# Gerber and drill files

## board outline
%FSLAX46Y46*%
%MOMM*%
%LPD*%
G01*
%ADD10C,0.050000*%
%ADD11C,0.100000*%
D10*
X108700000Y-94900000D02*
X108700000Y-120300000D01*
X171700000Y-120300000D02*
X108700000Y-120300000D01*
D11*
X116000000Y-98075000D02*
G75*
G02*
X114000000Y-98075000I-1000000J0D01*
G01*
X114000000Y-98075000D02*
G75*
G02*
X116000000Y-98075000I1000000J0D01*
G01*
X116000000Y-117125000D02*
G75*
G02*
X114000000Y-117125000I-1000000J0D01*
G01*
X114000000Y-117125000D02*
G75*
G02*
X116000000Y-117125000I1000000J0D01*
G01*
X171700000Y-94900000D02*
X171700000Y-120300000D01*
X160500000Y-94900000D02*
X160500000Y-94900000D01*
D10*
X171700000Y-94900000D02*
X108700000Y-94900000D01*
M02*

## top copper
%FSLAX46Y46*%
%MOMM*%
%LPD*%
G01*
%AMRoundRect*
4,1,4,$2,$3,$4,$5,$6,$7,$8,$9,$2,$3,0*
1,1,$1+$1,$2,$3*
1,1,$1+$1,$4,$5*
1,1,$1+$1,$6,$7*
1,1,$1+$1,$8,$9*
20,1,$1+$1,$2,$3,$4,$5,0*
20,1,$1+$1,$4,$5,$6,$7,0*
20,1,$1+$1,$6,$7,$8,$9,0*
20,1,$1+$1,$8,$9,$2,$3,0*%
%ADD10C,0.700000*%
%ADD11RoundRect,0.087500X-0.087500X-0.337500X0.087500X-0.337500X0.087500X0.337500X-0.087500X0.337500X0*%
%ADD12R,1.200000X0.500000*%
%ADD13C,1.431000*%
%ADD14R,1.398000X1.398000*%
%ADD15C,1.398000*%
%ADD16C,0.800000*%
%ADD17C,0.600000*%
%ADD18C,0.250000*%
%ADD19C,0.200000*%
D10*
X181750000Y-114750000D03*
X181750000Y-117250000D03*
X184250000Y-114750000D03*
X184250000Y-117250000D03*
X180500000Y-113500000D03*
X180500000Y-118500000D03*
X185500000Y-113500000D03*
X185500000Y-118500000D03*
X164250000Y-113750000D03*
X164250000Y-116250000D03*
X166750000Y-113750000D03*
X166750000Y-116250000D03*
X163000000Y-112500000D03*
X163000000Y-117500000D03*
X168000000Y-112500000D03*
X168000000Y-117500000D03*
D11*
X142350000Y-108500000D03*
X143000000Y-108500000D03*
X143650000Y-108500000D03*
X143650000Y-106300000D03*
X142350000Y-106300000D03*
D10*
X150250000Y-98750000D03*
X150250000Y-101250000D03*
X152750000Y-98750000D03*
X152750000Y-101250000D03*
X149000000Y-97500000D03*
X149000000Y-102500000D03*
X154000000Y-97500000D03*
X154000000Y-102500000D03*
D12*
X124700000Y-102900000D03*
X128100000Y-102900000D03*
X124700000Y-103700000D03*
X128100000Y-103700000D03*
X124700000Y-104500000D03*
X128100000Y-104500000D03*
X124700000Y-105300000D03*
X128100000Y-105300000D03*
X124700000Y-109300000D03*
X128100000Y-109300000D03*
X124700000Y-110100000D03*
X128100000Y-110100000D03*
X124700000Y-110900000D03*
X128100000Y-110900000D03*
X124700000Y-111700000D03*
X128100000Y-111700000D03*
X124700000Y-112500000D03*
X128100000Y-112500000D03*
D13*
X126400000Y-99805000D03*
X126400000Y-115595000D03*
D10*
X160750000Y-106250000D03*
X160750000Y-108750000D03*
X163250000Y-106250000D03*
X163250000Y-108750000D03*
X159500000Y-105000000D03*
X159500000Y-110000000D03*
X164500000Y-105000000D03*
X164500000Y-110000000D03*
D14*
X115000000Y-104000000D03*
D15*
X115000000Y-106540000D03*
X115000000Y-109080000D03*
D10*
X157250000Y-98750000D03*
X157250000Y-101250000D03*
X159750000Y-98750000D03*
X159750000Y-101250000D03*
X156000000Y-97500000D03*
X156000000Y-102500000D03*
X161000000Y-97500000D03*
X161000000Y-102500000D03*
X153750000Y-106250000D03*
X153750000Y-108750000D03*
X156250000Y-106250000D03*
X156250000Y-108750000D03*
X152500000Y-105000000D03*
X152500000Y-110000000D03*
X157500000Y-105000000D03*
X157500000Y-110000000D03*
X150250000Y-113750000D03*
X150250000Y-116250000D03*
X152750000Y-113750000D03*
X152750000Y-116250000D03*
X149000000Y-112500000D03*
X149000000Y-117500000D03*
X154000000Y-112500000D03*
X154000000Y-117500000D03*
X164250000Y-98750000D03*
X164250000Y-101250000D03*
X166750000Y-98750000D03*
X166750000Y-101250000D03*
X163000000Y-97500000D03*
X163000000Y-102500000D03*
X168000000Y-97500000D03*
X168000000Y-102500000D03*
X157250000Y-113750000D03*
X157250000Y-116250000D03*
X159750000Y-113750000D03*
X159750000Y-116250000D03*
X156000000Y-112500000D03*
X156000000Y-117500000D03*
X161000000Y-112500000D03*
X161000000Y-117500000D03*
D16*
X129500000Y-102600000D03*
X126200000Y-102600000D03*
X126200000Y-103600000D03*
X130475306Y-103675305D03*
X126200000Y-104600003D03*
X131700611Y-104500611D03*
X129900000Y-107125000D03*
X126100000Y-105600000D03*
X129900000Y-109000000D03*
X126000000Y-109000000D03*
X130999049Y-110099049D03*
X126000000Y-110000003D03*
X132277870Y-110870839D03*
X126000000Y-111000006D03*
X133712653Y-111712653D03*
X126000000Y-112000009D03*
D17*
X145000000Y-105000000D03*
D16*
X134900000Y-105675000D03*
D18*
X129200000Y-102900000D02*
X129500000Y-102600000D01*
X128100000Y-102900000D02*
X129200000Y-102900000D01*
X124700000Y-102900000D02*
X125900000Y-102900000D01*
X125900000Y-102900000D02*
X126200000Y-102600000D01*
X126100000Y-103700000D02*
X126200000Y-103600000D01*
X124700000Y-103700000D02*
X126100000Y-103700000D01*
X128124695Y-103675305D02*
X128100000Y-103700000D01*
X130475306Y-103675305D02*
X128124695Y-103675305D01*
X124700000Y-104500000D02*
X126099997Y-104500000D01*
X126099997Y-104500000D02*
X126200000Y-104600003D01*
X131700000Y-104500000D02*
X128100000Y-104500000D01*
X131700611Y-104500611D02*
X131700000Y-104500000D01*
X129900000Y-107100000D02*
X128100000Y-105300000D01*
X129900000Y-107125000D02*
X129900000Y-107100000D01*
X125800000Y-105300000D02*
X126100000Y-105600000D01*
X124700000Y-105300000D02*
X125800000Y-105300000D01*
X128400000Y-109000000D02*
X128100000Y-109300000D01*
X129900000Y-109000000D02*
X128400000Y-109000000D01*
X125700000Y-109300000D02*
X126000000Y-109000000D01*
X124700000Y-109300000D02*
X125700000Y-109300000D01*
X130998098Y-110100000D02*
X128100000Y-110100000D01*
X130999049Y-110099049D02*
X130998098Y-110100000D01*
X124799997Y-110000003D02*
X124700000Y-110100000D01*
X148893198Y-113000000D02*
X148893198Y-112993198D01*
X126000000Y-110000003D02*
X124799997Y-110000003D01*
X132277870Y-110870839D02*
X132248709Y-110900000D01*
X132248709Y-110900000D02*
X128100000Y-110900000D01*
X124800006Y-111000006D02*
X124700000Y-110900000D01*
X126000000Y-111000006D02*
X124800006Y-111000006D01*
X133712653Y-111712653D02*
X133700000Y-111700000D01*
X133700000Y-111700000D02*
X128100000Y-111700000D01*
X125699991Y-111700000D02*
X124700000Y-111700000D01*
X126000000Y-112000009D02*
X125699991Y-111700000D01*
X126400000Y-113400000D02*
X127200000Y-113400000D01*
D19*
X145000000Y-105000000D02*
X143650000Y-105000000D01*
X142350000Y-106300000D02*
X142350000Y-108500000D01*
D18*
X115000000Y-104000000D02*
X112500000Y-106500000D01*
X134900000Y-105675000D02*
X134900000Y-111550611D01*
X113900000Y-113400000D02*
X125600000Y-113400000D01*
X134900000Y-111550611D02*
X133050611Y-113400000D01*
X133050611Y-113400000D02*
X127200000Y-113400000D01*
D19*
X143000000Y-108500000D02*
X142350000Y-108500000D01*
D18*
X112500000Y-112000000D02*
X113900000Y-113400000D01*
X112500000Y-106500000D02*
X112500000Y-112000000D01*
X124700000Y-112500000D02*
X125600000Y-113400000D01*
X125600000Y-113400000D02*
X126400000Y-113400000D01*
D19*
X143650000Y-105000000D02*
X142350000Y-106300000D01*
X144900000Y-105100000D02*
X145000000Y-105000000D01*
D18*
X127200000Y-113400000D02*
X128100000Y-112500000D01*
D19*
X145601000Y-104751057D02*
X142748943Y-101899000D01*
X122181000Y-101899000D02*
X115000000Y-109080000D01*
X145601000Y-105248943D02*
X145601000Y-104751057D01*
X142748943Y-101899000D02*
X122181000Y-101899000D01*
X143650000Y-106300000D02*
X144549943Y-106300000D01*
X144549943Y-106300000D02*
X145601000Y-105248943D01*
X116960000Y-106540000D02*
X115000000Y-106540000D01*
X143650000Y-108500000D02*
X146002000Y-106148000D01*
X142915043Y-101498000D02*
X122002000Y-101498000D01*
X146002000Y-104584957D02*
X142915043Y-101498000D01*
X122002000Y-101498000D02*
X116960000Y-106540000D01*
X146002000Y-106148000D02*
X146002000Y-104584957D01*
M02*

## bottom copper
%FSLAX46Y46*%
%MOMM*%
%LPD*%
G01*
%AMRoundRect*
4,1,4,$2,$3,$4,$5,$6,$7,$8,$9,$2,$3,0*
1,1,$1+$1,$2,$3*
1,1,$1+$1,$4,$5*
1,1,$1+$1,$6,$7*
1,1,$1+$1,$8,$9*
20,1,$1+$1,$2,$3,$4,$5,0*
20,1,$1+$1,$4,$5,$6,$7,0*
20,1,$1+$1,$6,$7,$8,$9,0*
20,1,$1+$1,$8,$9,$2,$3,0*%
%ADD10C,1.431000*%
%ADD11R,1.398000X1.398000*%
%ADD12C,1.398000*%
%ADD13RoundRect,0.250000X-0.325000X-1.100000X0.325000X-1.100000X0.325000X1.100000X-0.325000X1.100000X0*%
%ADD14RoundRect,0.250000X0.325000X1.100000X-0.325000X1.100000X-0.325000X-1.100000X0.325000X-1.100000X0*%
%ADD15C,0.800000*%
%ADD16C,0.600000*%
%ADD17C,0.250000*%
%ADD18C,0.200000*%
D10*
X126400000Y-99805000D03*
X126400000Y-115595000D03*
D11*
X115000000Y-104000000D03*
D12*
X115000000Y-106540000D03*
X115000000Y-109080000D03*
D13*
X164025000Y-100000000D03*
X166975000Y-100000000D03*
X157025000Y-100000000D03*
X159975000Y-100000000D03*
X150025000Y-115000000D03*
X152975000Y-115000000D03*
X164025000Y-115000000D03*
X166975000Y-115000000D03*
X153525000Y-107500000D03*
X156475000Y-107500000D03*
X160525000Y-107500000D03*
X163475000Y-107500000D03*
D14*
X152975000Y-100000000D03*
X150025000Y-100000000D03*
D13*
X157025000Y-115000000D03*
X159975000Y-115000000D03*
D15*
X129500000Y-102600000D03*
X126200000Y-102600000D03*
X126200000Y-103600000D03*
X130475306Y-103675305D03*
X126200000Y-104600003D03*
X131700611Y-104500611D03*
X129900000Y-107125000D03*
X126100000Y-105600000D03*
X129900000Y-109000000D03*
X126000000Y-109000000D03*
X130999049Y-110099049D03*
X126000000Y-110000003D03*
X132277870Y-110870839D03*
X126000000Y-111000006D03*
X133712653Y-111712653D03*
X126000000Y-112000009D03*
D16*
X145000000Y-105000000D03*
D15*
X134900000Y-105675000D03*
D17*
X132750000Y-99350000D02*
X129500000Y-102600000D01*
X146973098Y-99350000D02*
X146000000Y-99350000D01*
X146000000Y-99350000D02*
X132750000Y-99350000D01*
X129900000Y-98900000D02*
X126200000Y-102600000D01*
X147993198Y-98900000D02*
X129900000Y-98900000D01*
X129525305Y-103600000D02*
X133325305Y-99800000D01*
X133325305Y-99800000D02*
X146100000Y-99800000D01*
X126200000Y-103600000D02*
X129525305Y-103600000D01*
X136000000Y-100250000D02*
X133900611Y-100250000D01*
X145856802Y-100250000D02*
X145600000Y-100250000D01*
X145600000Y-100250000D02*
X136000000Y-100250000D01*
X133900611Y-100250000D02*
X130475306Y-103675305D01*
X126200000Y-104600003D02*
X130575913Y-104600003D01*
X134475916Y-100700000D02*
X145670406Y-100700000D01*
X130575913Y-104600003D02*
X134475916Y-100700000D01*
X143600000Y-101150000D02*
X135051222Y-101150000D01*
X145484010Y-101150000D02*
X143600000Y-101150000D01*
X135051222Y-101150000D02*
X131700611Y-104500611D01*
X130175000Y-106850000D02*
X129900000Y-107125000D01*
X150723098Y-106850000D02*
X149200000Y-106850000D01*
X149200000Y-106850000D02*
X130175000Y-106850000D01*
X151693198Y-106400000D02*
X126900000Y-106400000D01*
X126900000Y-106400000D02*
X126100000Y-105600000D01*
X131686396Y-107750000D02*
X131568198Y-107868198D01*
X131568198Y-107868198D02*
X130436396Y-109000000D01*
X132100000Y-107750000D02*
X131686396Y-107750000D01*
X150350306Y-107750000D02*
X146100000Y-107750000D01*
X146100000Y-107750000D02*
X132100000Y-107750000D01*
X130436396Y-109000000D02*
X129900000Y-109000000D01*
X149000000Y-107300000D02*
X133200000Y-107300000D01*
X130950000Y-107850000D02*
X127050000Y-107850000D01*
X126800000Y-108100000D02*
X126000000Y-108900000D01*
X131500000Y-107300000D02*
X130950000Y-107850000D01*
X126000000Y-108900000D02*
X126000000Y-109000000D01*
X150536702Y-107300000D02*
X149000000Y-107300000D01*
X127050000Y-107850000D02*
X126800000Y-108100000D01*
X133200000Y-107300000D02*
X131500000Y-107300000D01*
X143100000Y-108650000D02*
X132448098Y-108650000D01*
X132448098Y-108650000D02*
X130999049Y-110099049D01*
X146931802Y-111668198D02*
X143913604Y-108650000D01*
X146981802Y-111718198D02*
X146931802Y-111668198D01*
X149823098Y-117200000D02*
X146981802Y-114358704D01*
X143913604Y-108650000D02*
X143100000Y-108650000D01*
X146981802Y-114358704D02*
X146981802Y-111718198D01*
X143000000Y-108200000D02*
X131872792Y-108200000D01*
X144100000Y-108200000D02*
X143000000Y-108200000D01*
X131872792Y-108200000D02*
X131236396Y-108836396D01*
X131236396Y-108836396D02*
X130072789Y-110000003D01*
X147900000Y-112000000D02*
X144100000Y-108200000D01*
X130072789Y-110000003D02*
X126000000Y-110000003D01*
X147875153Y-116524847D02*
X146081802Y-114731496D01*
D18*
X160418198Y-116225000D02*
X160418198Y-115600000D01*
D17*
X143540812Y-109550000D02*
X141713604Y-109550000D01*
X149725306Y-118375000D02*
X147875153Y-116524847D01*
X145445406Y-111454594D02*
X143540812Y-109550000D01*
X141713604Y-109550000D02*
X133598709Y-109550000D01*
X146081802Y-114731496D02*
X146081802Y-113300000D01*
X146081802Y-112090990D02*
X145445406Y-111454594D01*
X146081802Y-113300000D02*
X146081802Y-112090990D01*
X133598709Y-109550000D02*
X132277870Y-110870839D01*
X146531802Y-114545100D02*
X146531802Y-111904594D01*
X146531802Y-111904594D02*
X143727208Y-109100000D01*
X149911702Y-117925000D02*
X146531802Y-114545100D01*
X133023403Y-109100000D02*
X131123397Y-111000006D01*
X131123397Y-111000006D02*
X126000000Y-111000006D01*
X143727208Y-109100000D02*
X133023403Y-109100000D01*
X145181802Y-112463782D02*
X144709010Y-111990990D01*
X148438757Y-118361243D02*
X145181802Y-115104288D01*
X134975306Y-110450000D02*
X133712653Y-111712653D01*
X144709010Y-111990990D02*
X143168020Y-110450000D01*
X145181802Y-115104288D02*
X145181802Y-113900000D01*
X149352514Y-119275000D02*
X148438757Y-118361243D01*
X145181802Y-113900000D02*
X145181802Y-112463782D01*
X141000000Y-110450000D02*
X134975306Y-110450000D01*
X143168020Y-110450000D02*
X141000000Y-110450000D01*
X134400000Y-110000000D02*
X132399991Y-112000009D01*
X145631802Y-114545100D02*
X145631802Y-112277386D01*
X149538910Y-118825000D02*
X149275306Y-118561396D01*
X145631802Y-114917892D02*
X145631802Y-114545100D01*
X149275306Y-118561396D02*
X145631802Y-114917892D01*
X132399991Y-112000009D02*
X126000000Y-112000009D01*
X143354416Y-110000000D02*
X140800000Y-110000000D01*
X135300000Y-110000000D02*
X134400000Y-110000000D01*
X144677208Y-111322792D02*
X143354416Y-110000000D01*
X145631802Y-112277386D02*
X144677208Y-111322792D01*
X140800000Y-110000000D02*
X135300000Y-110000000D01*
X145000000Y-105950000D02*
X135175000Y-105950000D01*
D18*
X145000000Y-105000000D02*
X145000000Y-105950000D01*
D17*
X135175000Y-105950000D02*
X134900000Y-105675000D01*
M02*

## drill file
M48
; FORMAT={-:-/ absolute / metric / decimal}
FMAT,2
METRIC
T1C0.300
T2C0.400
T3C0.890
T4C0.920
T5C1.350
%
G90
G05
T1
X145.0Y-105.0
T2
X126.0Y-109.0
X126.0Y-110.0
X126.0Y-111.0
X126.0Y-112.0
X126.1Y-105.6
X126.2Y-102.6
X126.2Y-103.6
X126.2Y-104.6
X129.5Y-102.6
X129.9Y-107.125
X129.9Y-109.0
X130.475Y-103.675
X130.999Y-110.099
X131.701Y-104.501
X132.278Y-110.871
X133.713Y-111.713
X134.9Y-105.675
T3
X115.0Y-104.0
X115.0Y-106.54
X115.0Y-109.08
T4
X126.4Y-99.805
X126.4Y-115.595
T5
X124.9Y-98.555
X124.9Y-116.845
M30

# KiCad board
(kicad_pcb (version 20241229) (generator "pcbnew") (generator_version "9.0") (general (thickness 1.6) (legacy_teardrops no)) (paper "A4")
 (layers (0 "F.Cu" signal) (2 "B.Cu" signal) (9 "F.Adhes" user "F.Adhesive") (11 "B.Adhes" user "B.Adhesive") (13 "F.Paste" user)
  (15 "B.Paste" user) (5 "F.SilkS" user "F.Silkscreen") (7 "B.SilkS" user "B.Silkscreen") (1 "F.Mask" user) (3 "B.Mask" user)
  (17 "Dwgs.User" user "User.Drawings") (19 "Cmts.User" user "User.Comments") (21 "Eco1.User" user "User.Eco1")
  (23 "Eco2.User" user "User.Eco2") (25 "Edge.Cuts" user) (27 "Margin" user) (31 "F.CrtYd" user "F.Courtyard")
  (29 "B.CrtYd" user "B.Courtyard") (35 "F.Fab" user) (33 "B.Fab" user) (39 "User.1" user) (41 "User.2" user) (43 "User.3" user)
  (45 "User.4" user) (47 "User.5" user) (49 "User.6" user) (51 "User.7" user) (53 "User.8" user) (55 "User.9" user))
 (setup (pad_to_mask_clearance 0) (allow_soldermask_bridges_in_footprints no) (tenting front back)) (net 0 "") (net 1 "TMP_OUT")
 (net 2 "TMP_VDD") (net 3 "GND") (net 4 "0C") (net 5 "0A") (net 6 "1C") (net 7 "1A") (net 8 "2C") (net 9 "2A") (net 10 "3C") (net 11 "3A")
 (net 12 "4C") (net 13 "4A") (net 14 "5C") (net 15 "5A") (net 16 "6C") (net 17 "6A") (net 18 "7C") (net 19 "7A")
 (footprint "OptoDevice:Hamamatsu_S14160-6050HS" (layer "F.Cu") (at 183 116)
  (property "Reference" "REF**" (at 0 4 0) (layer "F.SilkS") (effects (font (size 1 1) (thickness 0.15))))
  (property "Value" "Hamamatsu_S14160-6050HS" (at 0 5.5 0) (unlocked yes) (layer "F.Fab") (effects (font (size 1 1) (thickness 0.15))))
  (pad "A" smd circle (at -1.25 -1.25) (size 0.7 0.7) (layers "F.Cu" "F.Mask" "F.Paste"))
  (pad "A" smd circle (at -1.25 1.25) (size 0.7 0.7) (layers "F.Cu" "F.Mask" "F.Paste"))
  (pad "A" smd circle (at 1.25 -1.25) (size 0.7 0.7) (layers "F.Cu" "F.Mask" "F.Paste"))
  (pad "A" smd circle (at 1.25 1.25) (size 0.7 0.7) (layers "F.Cu" "F.Mask" "F.Paste"))
  (pad "K" smd circle (at -2.5 -2.5) (size 0.7 0.7) (layers "F.Cu" "F.Mask" "F.Paste"))
  (pad "K" smd circle (at -2.5 2.5) (size 0.7 0.7) (layers "F.Cu" "F.Mask" "F.Paste"))
  (pad "K" smd circle (at 2.5 -2.5) (size 0.7 0.7) (layers "F.Cu" "F.Mask" "F.Paste"))
  (pad "K" smd circle (at 2.5 2.5) (size 0.7 0.7) (layers "F.Cu" "F.Mask" "F.Paste")))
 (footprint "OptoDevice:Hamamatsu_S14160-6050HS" (layer "F.Cu") (at 165.5 115)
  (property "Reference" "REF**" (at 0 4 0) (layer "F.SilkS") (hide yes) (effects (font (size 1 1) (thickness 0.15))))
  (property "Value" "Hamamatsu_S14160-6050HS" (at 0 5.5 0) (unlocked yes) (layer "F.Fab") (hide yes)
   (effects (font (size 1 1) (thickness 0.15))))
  (pad "A" smd circle (at -1.25 -1.25) (size 0.7 0.7) (layers "F.Cu" "F.Mask" "F.Paste"))
  (pad "A" smd circle (at -1.25 1.25) (size 0.7 0.7) (layers "F.Cu" "F.Mask" "F.Paste"))
  (pad "A" smd circle (at 1.25 -1.25) (size 0.7 0.7) (layers "F.Cu" "F.Mask" "F.Paste"))
  (pad "A" smd circle (at 1.25 1.25) (size 0.7 0.7) (layers "F.Cu" "F.Mask" "F.Paste"))
  (pad "K" smd circle (at -2.5 -2.5) (size 0.7 0.7) (layers "F.Cu" "F.Mask" "F.Paste"))
  (pad "K" smd circle (at -2.5 2.5) (size 0.7 0.7) (layers "F.Cu" "F.Mask" "F.Paste"))
  (pad "K" smd circle (at 2.5 -2.5) (size 0.7 0.7) (layers "F.Cu" "F.Mask" "F.Paste"))
  (pad "K" smd circle (at 2.5 2.5) (size 0.7 0.7) (layers "F.Cu" "F.Mask" "F.Paste")))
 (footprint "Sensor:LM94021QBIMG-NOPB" (layer "F.Cu") (at 143 107.4)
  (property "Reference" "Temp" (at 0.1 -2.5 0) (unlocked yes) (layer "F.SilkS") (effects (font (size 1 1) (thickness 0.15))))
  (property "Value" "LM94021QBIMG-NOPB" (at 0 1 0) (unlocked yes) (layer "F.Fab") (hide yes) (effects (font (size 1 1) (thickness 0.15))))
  (pad "1" smd roundrect (at -0.65 1.1) (size 0.35 0.85) (layers "F.Cu" "F.Mask" "F.Paste") (roundrect_rratio 0.25))
  (pad "2" smd roundrect (at 0 1.1) (size 0.35 0.85) (layers "F.Cu" "F.Mask" "F.Paste") (roundrect_rratio 0.25))
  (pad "3" smd roundrect (at 0.65 1.1) (size 0.35 0.85) (layers "F.Cu" "F.Mask" "F.Paste") (roundrect_rratio 0.25) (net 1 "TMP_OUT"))
  (pad "4" smd roundrect (at 0.65 -1.1) (size 0.35 0.85) (layers "F.Cu" "F.Mask" "F.Paste") (roundrect_rratio 0.25) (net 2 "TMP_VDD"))
  (pad "5" smd roundrect (at -0.65 -1.1) (size 0.35 0.85) (layers "F.Cu" "F.Mask" "F.Paste") (roundrect_rratio 0.25) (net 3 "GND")))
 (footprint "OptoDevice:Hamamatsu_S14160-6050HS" (layer "F.Cu") (at 151.5 100)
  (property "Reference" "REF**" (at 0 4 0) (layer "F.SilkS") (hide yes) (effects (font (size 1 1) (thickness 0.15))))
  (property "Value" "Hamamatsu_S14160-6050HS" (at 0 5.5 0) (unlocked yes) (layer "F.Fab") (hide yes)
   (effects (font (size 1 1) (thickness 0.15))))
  (pad "A" smd circle (at -1.25 -1.25) (size 0.7 0.7) (layers "F.Cu" "F.Mask" "F.Paste") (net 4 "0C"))
  (pad "A" smd circle (at -1.25 1.25) (size 0.7 0.7) (layers "F.Cu" "F.Mask" "F.Paste") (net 4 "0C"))
  (pad "A" smd circle (at 1.25 -1.25) (size 0.7 0.7) (layers "F.Cu" "F.Mask" "F.Paste") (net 4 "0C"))
  (pad "A" smd circle (at 1.25 1.25) (size 0.7 0.7) (layers "F.Cu" "F.Mask" "F.Paste") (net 4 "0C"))
  (pad "K" smd circle (at -2.5 -2.5) (size 0.7 0.7) (layers "F.Cu" "F.Mask" "F.Paste") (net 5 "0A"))
  (pad "K" smd circle (at -2.5 2.5) (size 0.7 0.7) (layers "F.Cu" "F.Mask" "F.Paste") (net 5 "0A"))
  (pad "K" smd circle (at 2.5 -2.5) (size 0.7 0.7) (layers "F.Cu" "F.Mask" "F.Paste") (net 5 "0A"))
  (pad "K" smd circle (at 2.5 2.5) (size 0.7 0.7) (layers "F.Cu" "F.Mask" "F.Paste") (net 5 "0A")))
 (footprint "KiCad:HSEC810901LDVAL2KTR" (layer "F.Cu") (at 126.4 107.7 -90)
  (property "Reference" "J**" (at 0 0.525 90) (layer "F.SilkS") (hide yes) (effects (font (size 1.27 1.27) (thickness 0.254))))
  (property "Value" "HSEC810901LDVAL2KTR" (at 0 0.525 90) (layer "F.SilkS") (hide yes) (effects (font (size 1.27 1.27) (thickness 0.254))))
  (pad "" np_thru_hole circle (at -9.145 1.5 270) (size 1.35 1.35) (drill 1.35) (layers "*.Cu" "*.Mask"))
  (pad "" np_thru_hole circle (at 9.145 1.5 270) (size 1.35 1.35) (drill 1.35) (layers "*.Cu" "*.Mask"))
  (pad "1" smd rect (at -4.8 1.7 270) (size 0.5 1.2) (layers "F.Cu" "F.Mask" "F.Paste") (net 4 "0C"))
  (pad "2" smd rect (at -4.8 -1.7 270) (size 0.5 1.2) (layers "F.Cu" "F.Mask" "F.Paste") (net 5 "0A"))
  (pad "3" smd rect (at -4 1.7 270) (size 0.5 1.2) (layers "F.Cu" "F.Mask" "F.Paste") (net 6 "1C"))
  (pad "4" smd rect (at -4 -1.7 270) (size 0.5 1.2) (layers "F.Cu" "F.Mask" "F.Paste") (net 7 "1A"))
  (pad "5" smd rect (at -3.2 1.7 270) (size 0.5 1.2) (layers "F.Cu" "F.Mask" "F.Paste") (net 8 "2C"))
  (pad "6" smd rect (at -3.2 -1.7 270) (size 0.5 1.2) (layers "F.Cu" "F.Mask" "F.Paste") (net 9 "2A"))
  (pad "7" smd rect (at -2.4 1.7 270) (size 0.5 1.2) (layers "F.Cu" "F.Mask" "F.Paste") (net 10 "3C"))
  (pad "8" smd rect (at -2.4 -1.7 270) (size 0.5 1.2) (layers "F.Cu" "F.Mask" "F.Paste") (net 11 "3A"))
  (pad "9" smd rect (at 1.6 1.7 270) (size 0.5 1.2) (layers "F.Cu" "F.Mask" "F.Paste") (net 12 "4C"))
  (pad "10" smd rect (at 1.6 -1.7 270) (size 0.5 1.2) (layers "F.Cu" "F.Mask" "F.Paste") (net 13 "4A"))
  (pad "11" smd rect (at 2.4 1.7 270) (size 0.5 1.2) (layers "F.Cu" "F.Mask" "F.Paste") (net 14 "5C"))
  (pad "12" smd rect (at 2.4 -1.7 270) (size 0.5 1.2) (layers "F.Cu" "F.Mask" "F.Paste") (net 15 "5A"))
  (pad "13" smd rect (at 3.2 1.7 270) (size 0.5 1.2) (layers "F.Cu" "F.Mask" "F.Paste") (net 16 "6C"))
  (pad "14" smd rect (at 3.2 -1.7 270) (size 0.5 1.2) (layers "F.Cu" "F.Mask" "F.Paste") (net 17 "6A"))
  (pad "15" smd rect (at 4 1.7 270) (size 0.5 1.2) (layers "F.Cu" "F.Mask" "F.Paste") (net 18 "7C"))
  (pad "16" smd rect (at 4 -1.7 270) (size 0.5 1.2) (layers "F.Cu" "F.Mask" "F.Paste") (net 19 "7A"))
  (pad "17" smd rect (at 4.8 1.7 270) (size 0.5 1.2) (layers "F.Cu" "F.Mask" "F.Paste") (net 3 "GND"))
  (pad "18" smd rect (at 4.8 -1.7 270) (size 0.5 1.2) (layers "F.Cu" "F.Mask" "F.Paste") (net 3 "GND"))
  (pad "MH1" thru_hole circle (at -7.895 0 270) (size 1.431 1.431) (drill 0.92) (layers "*.Cu" "*.Mask") (remove_unused_layers no))
  (pad "MH2" thru_hole circle (at 7.895 0 270) (size 1.431 1.431) (drill 0.92) (layers "*.Cu" "*.Mask") (remove_unused_layers no)))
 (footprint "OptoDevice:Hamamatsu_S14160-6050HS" (layer "F.Cu") (at 162 107.5)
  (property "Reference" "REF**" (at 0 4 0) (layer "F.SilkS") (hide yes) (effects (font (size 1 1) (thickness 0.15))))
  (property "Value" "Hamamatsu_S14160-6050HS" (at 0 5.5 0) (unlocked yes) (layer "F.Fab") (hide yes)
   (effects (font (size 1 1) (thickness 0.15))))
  (pad "A" smd circle (at -1.25 -1.25) (size 0.7 0.7) (layers "F.Cu" "F.Mask" "F.Paste"))
  (pad "A" smd circle (at -1.25 1.25) (size 0.7 0.7) (layers "F.Cu" "F.Mask" "F.Paste"))
  (pad "A" smd circle (at 1.25 -1.25) (size 0.7 0.7) (layers "F.Cu" "F.Mask" "F.Paste"))
  (pad "A" smd circle (at 1.25 1.25) (size 0.7 0.7) (layers "F.Cu" "F.Mask" "F.Paste"))
  (pad "K" smd circle (at -2.5 -2.5) (size 0.7 0.7) (layers "F.Cu" "F.Mask" "F.Paste"))
  (pad "K" smd circle (at -2.5 2.5) (size 0.7 0.7) (layers "F.Cu" "F.Mask" "F.Paste"))
  (pad "K" smd circle (at 2.5 -2.5) (size 0.7 0.7) (layers "F.Cu" "F.Mask" "F.Paste"))
  (pad "K" smd circle (at 2.5 2.5) (size 0.7 0.7) (layers "F.Cu" "F.Mask" "F.Paste")))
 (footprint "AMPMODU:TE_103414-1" (layer "F.Cu") (at 115 106.54 -90)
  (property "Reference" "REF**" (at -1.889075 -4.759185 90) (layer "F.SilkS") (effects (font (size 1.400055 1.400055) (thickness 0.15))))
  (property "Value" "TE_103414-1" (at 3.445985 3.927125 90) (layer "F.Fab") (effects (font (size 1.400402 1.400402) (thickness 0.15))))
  (pad "1" thru_hole rect (at -2.54 0 270) (size 1.398 1.398) (drill 0.89) (layers "*.Cu" "*.Mask") (remove_unused_layers no) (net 3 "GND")
   (solder_mask_margin 0.102))
  (pad "2" thru_hole circle (at 0 0 270) (size 1.398 1.398) (drill 0.89) (layers "*.Cu" "*.Mask") (remove_unused_layers no)
   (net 1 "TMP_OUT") (solder_mask_margin 0.102))
  (pad "3" thru_hole circle (at 2.54 0 270) (size 1.398 1.398) (drill 0.89) (layers "*.Cu" "*.Mask") (remove_unused_layers no)
   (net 2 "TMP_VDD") (solder_mask_margin 0.102)))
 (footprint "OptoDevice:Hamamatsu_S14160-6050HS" (layer "F.Cu") (at 158.5 100)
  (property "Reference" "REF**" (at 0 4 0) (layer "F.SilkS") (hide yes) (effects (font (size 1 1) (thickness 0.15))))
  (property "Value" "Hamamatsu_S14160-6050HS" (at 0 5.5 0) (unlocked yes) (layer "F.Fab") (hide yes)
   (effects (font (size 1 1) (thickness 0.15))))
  (pad "A" smd circle (at -1.25 -1.25) (size 0.7 0.7) (layers "F.Cu" "F.Mask" "F.Paste") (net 6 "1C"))
  (pad "A" smd circle (at -1.25 1.25) (size 0.7 0.7) (layers "F.Cu" "F.Mask" "F.Paste") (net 6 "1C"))
  (pad "A" smd circle (at 1.25 -1.25) (size 0.7 0.7) (layers "F.Cu" "F.Mask" "F.Paste") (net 6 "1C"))
  (pad "A" smd circle (at 1.25 1.25) (size 0.7 0.7) (layers "F.Cu" "F.Mask" "F.Paste") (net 6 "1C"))
  (pad "K" smd circle (at -2.5 -2.5) (size 0.7 0.7) (layers "F.Cu" "F.Mask" "F.Paste") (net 7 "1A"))
  (pad "K" smd circle (at -2.5 2.5) (size 0.7 0.7) (layers "F.Cu" "F.Mask" "F.Paste") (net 7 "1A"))
  (pad "K" smd circle (at 2.5 -2.5) (size 0.7 0.7) (layers "F.Cu" "F.Mask" "F.Paste") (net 7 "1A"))
  (pad "K" smd circle (at 2.5 2.5) (size 0.7 0.7) (layers "F.Cu" "F.Mask" "F.Paste") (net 7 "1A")))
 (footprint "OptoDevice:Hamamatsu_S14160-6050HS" (layer "F.Cu") (at 155 107.5)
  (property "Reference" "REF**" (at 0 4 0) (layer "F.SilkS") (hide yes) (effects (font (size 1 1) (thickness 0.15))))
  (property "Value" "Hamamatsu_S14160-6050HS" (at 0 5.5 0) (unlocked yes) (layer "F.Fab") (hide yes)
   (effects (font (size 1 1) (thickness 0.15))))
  (pad "A" smd circle (at -1.25 -1.25) (size 0.7 0.7) (layers "F.Cu" "F.Mask" "F.Paste") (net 10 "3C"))
  (pad "A" smd circle (at -1.25 1.25) (size 0.7 0.7) (layers "F.Cu" "F.Mask" "F.Paste") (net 10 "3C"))
  (pad "A" smd circle (at 1.25 -1.25) (size 0.7 0.7) (layers "F.Cu" "F.Mask" "F.Paste") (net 10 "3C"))
  (pad "A" smd circle (at 1.25 1.25) (size 0.7 0.7) (layers "F.Cu" "F.Mask" "F.Paste") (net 10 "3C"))
  (pad "K" smd circle (at -2.5 -2.5) (size 0.7 0.7) (layers "F.Cu" "F.Mask" "F.Paste") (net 11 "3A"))
  (pad "K" smd circle (at -2.5 2.5) (size 0.7 0.7) (layers "F.Cu" "F.Mask" "F.Paste") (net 11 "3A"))
  (pad "K" smd circle (at 2.5 -2.5) (size 0.7 0.7) (layers "F.Cu" "F.Mask" "F.Paste") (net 11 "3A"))
  (pad "K" smd circle (at 2.5 2.5) (size 0.7 0.7) (layers "F.Cu" "F.Mask" "F.Paste") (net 11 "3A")))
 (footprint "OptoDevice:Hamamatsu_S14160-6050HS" (layer "F.Cu") (at 151.5 115)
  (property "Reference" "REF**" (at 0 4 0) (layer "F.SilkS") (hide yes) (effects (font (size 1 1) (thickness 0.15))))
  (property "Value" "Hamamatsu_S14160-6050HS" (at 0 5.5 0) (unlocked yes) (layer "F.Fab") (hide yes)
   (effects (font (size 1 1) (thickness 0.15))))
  (pad "A" smd circle (at -1.25 -1.25) (size 0.7 0.7) (layers "F.Cu" "F.Mask" "F.Paste"))
  (pad "A" smd circle (at -1.25 1.25) (size 0.7 0.7) (layers "F.Cu" "F.Mask" "F.Paste"))
  (pad "A" smd circle (at 1.25 -1.25) (size 0.7 0.7) (layers "F.Cu" "F.Mask" "F.Paste"))
  (pad "A" smd circle (at 1.25 1.25) (size 0.7 0.7) (layers "F.Cu" "F.Mask" "F.Paste"))
  (pad "K" smd circle (at -2.5 -2.5) (size 0.7 0.7) (layers "F.Cu" "F.Mask" "F.Paste"))
  (pad "K" smd circle (at -2.5 2.5) (size 0.7 0.7) (layers "F.Cu" "F.Mask" "F.Paste"))
  (pad "K" smd circle (at 2.5 -2.5) (size 0.7 0.7) (layers "F.Cu" "F.Mask" "F.Paste"))
  (pad "K" smd circle (at 2.5 2.5) (size 0.7 0.7) (layers "F.Cu" "F.Mask" "F.Paste")))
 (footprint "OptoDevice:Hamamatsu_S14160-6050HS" (layer "F.Cu") (at 165.5 100)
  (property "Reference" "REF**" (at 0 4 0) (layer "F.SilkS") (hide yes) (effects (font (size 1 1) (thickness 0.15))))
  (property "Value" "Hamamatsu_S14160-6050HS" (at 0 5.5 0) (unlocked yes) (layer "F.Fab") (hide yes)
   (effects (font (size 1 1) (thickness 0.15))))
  (pad "A" smd circle (at -1.25 -1.25) (size 0.7 0.7) (layers "F.Cu" "F.Mask" "F.Paste") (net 8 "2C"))
  (pad "A" smd circle (at -1.25 1.25) (size 0.7 0.7) (layers "F.Cu" "F.Mask" "F.Paste") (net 8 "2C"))
  (pad "A" smd circle (at 1.25 -1.25) (size 0.7 0.7) (layers "F.Cu" "F.Mask" "F.Paste") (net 8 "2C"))
  (pad "A" smd circle (at 1.25 1.25) (size 0.7 0.7) (layers "F.Cu" "F.Mask" "F.Paste") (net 8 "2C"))
  (pad "K" smd circle (at -2.5 -2.5) (size 0.7 0.7) (layers "F.Cu" "F.Mask" "F.Paste") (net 9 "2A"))
  (pad "K" smd circle (at -2.5 2.5) (size 0.7 0.7) (layers "F.Cu" "F.Mask" "F.Paste") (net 9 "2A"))
  (pad "K" smd circle (at 2.5 -2.5) (size 0.7 0.7) (layers "F.Cu" "F.Mask" "F.Paste") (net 9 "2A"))
  (pad "K" smd circle (at 2.5 2.5) (size 0.7 0.7) (layers "F.Cu" "F.Mask" "F.Paste") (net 9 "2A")))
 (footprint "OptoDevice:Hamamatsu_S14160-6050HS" (layer "F.Cu") (at 158.5 115)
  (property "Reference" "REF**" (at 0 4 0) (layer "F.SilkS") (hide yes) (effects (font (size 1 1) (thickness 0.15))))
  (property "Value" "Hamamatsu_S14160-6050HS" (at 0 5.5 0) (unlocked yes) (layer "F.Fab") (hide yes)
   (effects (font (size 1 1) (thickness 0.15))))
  (pad "A" smd circle (at -1.25 -1.25) (size 0.7 0.7) (layers "F.Cu" "F.Mask" "F.Paste"))
  (pad "A" smd circle (at -1.25 1.25) (size 0.7 0.7) (layers "F.Cu" "F.Mask" "F.Paste"))
  (pad "A" smd circle (at 1.25 -1.25) (size 0.7 0.7) (layers "F.Cu" "F.Mask" "F.Paste"))
  (pad "A" smd circle (at 1.25 1.25) (size 0.7 0.7) (layers "F.Cu" "F.Mask" "F.Paste"))
  (pad "K" smd circle (at -2.5 -2.5) (size 0.7 0.7) (layers "F.Cu" "F.Mask" "F.Paste"))
  (pad "K" smd circle (at -2.5 2.5) (size 0.7 0.7) (layers "F.Cu" "F.Mask" "F.Paste"))
  (pad "K" smd circle (at 2.5 -2.5) (size 0.7 0.7) (layers "F.Cu" "F.Mask" "F.Paste"))
  (pad "K" smd circle (at 2.5 2.5) (size 0.7 0.7) (layers "F.Cu" "F.Mask" "F.Paste")))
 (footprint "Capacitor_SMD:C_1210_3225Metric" (layer "B.Cu") (at 165.5 100)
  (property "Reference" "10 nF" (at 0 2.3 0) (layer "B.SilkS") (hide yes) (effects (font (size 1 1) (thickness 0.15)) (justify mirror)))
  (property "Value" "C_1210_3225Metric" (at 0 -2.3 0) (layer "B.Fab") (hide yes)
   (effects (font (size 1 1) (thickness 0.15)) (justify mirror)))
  (pad "1" smd roundrect (at -1.475 0) (size 1.15 2.7) (layers "B.Cu" "B.Mask" "B.Paste") (roundrect_rratio 0.2173913043) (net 3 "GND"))
  (pad "2" smd roundrect (at 1.475 0) (size 1.15 2.7) (layers "B.Cu" "B.Mask" "B.Paste") (roundrect_rratio 0.2173913043) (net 9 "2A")))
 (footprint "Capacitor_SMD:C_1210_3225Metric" (layer "B.Cu") (at 158.5 100)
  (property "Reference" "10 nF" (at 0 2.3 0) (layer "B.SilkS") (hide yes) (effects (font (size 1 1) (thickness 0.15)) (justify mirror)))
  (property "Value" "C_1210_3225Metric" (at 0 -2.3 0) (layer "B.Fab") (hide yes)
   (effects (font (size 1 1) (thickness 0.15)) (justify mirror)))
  (pad "1" smd roundrect (at -1.475 0) (size 1.15 2.7) (layers "B.Cu" "B.Mask" "B.Paste") (roundrect_rratio 0.2173913043) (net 3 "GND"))
  (pad "2" smd roundrect (at 1.475 0) (size 1.15 2.7) (layers "B.Cu" "B.Mask" "B.Paste") (roundrect_rratio 0.2173913043) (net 7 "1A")))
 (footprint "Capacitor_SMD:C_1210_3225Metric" (layer "B.Cu") (at 151.5 115)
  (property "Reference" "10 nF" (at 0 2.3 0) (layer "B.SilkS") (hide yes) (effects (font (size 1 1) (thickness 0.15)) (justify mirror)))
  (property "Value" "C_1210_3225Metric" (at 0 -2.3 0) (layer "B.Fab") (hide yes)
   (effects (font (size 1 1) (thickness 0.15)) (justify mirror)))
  (pad "1" smd roundrect (at -1.475 0) (size 1.15 2.7) (layers "B.Cu" "B.Mask" "B.Paste") (roundrect_rratio 0.2173913043) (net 3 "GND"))
  (pad "2" smd roundrect (at 1.475 0) (size 1.15 2.7) (layers "B.Cu" "B.Mask" "B.Paste") (roundrect_rratio 0.2173913043) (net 15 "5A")))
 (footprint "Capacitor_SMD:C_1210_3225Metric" (layer "B.Cu") (at 165.5 115)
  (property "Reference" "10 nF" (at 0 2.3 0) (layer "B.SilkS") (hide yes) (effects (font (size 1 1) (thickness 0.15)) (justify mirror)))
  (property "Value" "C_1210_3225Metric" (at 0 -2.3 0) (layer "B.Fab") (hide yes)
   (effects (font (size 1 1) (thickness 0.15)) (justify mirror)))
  (pad "1" smd roundrect (at -1.475 0) (size 1.15 2.7) (layers "B.Cu" "B.Mask" "B.Paste") (roundrect_rratio 0.2173913043) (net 3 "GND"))
  (pad "2" smd roundrect (at 1.475 0) (size 1.15 2.7) (layers "B.Cu" "B.Mask" "B.Paste") (roundrect_rratio 0.2173913043) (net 19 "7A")))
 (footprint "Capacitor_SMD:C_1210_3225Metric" (layer "B.Cu") (at 155 107.5)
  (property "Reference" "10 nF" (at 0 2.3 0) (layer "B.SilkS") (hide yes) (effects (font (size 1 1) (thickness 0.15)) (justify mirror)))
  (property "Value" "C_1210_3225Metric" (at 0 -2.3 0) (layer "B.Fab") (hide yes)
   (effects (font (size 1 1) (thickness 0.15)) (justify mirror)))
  (pad "1" smd roundrect (at -1.475 0) (size 1.15 2.7) (layers "B.Cu" "B.Mask" "B.Paste") (roundrect_rratio 0.2173913043) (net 3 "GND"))
  (pad "2" smd roundrect (at 1.475 0) (size 1.15 2.7) (layers "B.Cu" "B.Mask" "B.Paste") (roundrect_rratio 0.2173913043) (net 11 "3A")))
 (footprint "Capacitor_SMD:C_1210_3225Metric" (layer "B.Cu") (at 162 107.5)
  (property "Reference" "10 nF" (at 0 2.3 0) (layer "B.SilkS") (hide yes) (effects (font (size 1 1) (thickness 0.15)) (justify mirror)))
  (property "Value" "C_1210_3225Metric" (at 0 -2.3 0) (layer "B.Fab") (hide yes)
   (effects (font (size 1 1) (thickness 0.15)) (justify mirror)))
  (pad "1" smd roundrect (at -1.475 0) (size 1.15 2.7) (layers "B.Cu" "B.Mask" "B.Paste") (roundrect_rratio 0.2173913043) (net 3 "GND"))
  (pad "2" smd roundrect (at 1.475 0) (size 1.15 2.7) (layers "B.Cu" "B.Mask" "B.Paste") (roundrect_rratio 0.2173913043) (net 13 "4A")))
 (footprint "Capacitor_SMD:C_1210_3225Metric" (layer "B.Cu") (at 151.5 100 180)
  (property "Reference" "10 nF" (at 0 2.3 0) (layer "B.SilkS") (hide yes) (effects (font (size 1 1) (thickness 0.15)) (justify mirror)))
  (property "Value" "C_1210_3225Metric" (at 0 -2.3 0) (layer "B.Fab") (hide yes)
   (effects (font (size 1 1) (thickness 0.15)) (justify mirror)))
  (pad "1" smd roundrect (at -1.475 0 180) (size 1.15 2.7) (layers "B.Cu" "B.Mask" "B.Paste") (roundrect_rratio 0.2173913043) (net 5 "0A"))
  (pad "2" smd roundrect (at 1.475 0 180) (size 1.15 2.7) (layers "B.Cu" "B.Mask" "B.Paste") (roundrect_rratio 0.2173913043) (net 3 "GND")))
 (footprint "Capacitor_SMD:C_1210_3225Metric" (layer "B.Cu") (at 158.5 115)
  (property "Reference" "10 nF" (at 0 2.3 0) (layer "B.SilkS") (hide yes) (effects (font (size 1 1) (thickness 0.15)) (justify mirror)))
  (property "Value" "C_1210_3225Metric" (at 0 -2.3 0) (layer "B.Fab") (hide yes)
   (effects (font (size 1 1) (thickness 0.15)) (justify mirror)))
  (pad "1" smd roundrect (at -1.475 0) (size 1.15 2.7) (layers "B.Cu" "B.Mask" "B.Paste") (roundrect_rratio 0.2173913043) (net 3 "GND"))
  (pad "2" smd roundrect (at 1.475 0) (size 1.15 2.7) (layers "B.Cu" "B.Mask" "B.Paste") (roundrect_rratio 0.2173913043) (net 17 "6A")))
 (gr_line (start 108.7 94.9) (end 108.7 120.3) (stroke (width 0.05) (type default)) (layer "Edge.Cuts"))
 (gr_line (start 171.7 120.3) (end 108.7 120.3) (stroke (width 0.05) (type solid)) (layer "Edge.Cuts"))
 (gr_circle (center 115 98.075) (end 116 98.075) (stroke (width 0.1) (type solid)) (fill no) (layer "Edge.Cuts"))
 (gr_circle (center 115 117.125) (end 116 117.125) (stroke (width 0.1) (type solid)) (fill no) (layer "Edge.Cuts"))
 (gr_line (start 171.7 94.9) (end 171.7 120.3) (stroke (width 0.1) (type default)) (layer "Edge.Cuts"))
 (gr_line (start 160.5 94.9) (end 160.5 94.9) (stroke (width 0.1) (type default)) (layer "Edge.Cuts"))
 (gr_line (start 171.7 94.9) (end 108.7 94.9) (stroke (width 0.05) (type solid)) (layer "Edge.Cuts"))
 (segment (start 129.2 102.9) (end 129.5 102.6) (width 0.25) (layer "F.Cu") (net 5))
 (segment (start 128.1 102.9) (end 129.2 102.9) (width 0.25) (layer "F.Cu") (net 5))
 (via (at 129.5 102.6) (size 0.8) (drill 0.4) (layers "F.Cu" "B.Cu") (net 5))
 (segment (start 132.75 99.35) (end 129.5 102.6) (width 0.25) (layer "B.Cu") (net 5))
 (segment (start 146.973098 99.35) (end 146 99.35) (width 0.25) (layer "B.Cu") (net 5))
 (segment (start 146 99.35) (end 132.75 99.35) (width 0.25) (layer "B.Cu") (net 5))
 (segment (start 124.7 102.9) (end 125.9 102.9) (width 0.25) (layer "F.Cu") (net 4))
 (segment (start 125.9 102.9) (end 126.2 102.6) (width 0.25) (layer "F.Cu") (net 4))
 (via (at 126.2 102.6) (size 0.8) (drill 0.4) (layers "F.Cu" "B.Cu") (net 4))
 (segment (start 129.9 98.9) (end 126.2 102.6) (width 0.25) (layer "B.Cu") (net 4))
 (segment (start 147.993198 98.9) (end 129.9 98.9) (width 0.25) (layer "B.Cu") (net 4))
 (segment (start 126.1 103.7) (end 126.2 103.6) (width 0.25) (layer "F.Cu") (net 6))
 (segment (start 124.7 103.7) (end 126.1 103.7) (width 0.25) (layer "F.Cu") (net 6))
 (via (at 126.2 103.6) (size 0.8) (drill 0.4) (layers "F.Cu" "B.Cu") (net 6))
 (segment (start 129.525305 103.6) (end 133.325305 99.8) (width 0.25) (layer "B.Cu") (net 6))
 (segment (start 133.325305 99.8) (end 146.1 99.8) (width 0.25) (layer "B.Cu") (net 6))
 (segment (start 126.2 103.6) (end 129.525305 103.6) (width 0.25) (layer "B.Cu") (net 6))
 (segment (start 128.124695 103.675305) (end 128.1 103.7) (width 0.25) (layer "F.Cu") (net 7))
 (segment (start 130.475306 103.675305) (end 128.124695 103.675305) (width 0.25) (layer "F.Cu") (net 7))
 (via (at 130.475306 103.675305) (size 0.8) (drill 0.4) (layers "F.Cu" "B.Cu") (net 7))
 (segment (start 136 100.25) (end 133.900611 100.25) (width 0.25) (layer "B.Cu") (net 7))
 (segment (start 145.856802 100.25) (end 145.6 100.25) (width 0.25) (layer "B.Cu") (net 7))
 (segment (start 145.6 100.25) (end 136 100.25) (width 0.25) (layer "B.Cu") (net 7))
 (segment (start 133.900611 100.25) (end 130.475306 103.675305) (width 0.25) (layer "B.Cu") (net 7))
 (segment (start 124.7 104.5) (end 126.099997 104.5) (width 0.25) (layer "F.Cu") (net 8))
 (segment (start 126.099997 104.5) (end 126.2 104.600003) (width 0.25) (layer "F.Cu") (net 8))
 (via (at 126.2 104.600003) (size 0.8) (drill 0.4) (layers "F.Cu" "B.Cu") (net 8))
 (segment (start 126.2 104.600003) (end 130.575913 104.600003) (width 0.25) (layer "B.Cu") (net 8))
 (segment (start 134.475916 100.7) (end 145.670406 100.7) (width 0.25) (layer "B.Cu") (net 8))
 (segment (start 130.575913 104.600003) (end 134.475916 100.7) (width 0.25) (layer "B.Cu") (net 8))
 (segment (start 131.7 104.5) (end 128.1 104.5) (width 0.25) (layer "F.Cu") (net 9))
 (segment (start 131.700611 104.500611) (end 131.7 104.5) (width 0.25) (layer "F.Cu") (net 9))
 (via (at 131.700611 104.500611) (size 0.8) (drill 0.4) (layers "F.Cu" "B.Cu") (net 9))
 (segment (start 143.6 101.15) (end 135.051222 101.15) (width 0.25) (layer "B.Cu") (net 9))
 (segment (start 145.48401 101.15) (end 143.6 101.15) (width 0.25) (layer "B.Cu") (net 9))
 (segment (start 135.051222 101.15) (end 131.700611 104.500611) (width 0.25) (layer "B.Cu") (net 9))
 (segment (start 129.9 107.1) (end 128.1 105.3) (width 0.25) (layer "F.Cu") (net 11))
 (segment (start 129.9 107.125) (end 129.9 107.1) (width 0.25) (layer "F.Cu") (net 11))
 (via (at 129.9 107.125) (size 0.8) (drill 0.4) (layers "F.Cu" "B.Cu") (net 11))
 (segment (start 130.175 106.85) (end 129.9 107.125) (width 0.25) (layer "B.Cu") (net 11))
 (segment (start 150.723098 106.85) (end 149.2 106.85) (width 0.25) (layer "B.Cu") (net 11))
 (segment (start 149.2 106.85) (end 130.175 106.85) (width 0.25) (layer "B.Cu") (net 11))
 (segment (start 125.8 105.3) (end 126.1 105.6) (width 0.25) (layer "F.Cu") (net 10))
 (segment (start 124.7 105.3) (end 125.8 105.3) (width 0.25) (layer "F.Cu") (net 10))
 (via (at 126.1 105.6) (size 0.8) (drill 0.4) (layers "F.Cu" "B.Cu") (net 10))
 (segment (start 151.693198 106.4) (end 126.9 106.4) (width 0.25) (layer "B.Cu") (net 10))
 (segment (start 126.9 106.4) (end 126.1 105.6) (width 0.25) (layer "B.Cu") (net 10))
 (segment (start 128.4 109) (end 128.1 109.3) (width 0.25) (layer "F.Cu") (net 13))
 (segment (start 129.9 109) (end 128.4 109) (width 0.25) (layer "F.Cu") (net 13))
 (via (at 129.9 109) (size 0.8) (drill 0.4) (layers "F.Cu" "B.Cu") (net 13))
 (segment (start 131.686396 107.75) (end 131.568198 107.868198) (width 0.25) (layer "B.Cu") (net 13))
 (segment (start 131.568198 107.868198) (end 130.436396 109) (width 0.25) (layer "B.Cu") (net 13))
 (segment (start 132.1 107.75) (end 131.686396 107.75) (width 0.25) (layer "B.Cu") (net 13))
 (segment (start 150.350306 107.75) (end 146.1 107.75) (width 0.25) (layer "B.Cu") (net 13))
 (segment (start 146.1 107.75) (end 132.1 107.75) (width 0.25) (layer "B.Cu") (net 13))
 (segment (start 130.436396 109) (end 129.9 109) (width 0.25) (layer "B.Cu") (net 13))
 (segment (start 125.7 109.3) (end 126 109) (width 0.25) (layer "F.Cu") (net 12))
 (segment (start 124.7 109.3) (end 125.7 109.3) (width 0.25) (layer "F.Cu") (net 12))
 (via (at 126 109) (size 0.8) (drill 0.4) (layers "F.Cu" "B.Cu") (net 12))
 (segment (start 149 107.3) (end 133.2 107.3) (width 0.25) (layer "B.Cu") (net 12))
 (segment (start 130.95 107.85) (end 127.05 107.85) (width 0.25) (layer "B.Cu") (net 12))
 (segment (start 126.8 108.1) (end 126 108.9) (width 0.25) (layer "B.Cu") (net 12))
 (segment (start 131.5 107.3) (end 130.95 107.85) (width 0.25) (layer "B.Cu") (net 12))
 (segment (start 126 108.9) (end 126 109) (width 0.25) (layer "B.Cu") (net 12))
 (segment (start 150.536702 107.3) (end 149 107.3) (width 0.25) (layer "B.Cu") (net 12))
 (segment (start 127.05 107.85) (end 126.8 108.1) (width 0.25) (layer "B.Cu") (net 12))
 (segment (start 133.2 107.3) (end 131.5 107.3) (width 0.25) (layer "B.Cu") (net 12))
 (segment (start 130.998098 110.1) (end 128.1 110.1) (width 0.25) (layer "F.Cu") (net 15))
 (segment (start 130.999049 110.099049) (end 130.998098 110.1) (width 0.25) (layer "F.Cu") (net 15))
 (via (at 130.999049 110.099049) (size 0.8) (drill 0.4) (layers "F.Cu" "B.Cu") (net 15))
 (segment (start 143.1 108.65) (end 132.448098 108.65) (width 0.25) (layer "B.Cu") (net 15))
 (segment (start 132.448098 108.65) (end 130.999049 110.099049) (width 0.25) (layer "B.Cu") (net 15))
 (segment (start 146.931802 111.668198) (end 143.913604 108.65) (width 0.25) (layer "B.Cu") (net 15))
 (segment (start 146.981802 111.718198) (end 146.931802 111.668198) (width 0.25) (layer "B.Cu") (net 15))
 (segment (start 149.823098 117.2) (end 146.981802 114.358704) (width 0.25) (layer "B.Cu") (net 15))
 (segment (start 143.913604 108.65) (end 143.1 108.65) (width 0.25) (layer "B.Cu") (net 15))
 (segment (start 146.981802 114.358704) (end 146.981802 111.718198) (width 0.25) (layer "B.Cu") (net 15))
 (segment (start 124.799997 110.000003) (end 124.7 110.1) (width 0.25) (layer "F.Cu") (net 14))
 (segment (start 148.893198 113) (end 148.893198 112.993198) (width 0.25) (layer "F.Cu") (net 14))
 (segment (start 126 110.000003) (end 124.799997 110.000003) (width 0.25) (layer "F.Cu") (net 14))
 (via (at 126 110.000003) (size 0.8) (drill 0.4) (layers "F.Cu" "B.Cu") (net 14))
 (segment (start 143 108.2) (end 131.872792 108.2) (width 0.25) (layer "B.Cu") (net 14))
 (segment (start 144.1 108.2) (end 143 108.2) (width 0.25) (layer "B.Cu") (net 14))
 (segment (start 131.872792 108.2) (end 131.236396 108.836396) (width 0.25) (layer "B.Cu") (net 14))
 (segment (start 131.236396 108.836396) (end 130.072789 110.000003) (width 0.25) (layer "B.Cu") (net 14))
 (segment (start 147.9 112) (end 144.1 108.2) (width 0.25) (layer "B.Cu") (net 14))
 (segment (start 130.072789 110.000003) (end 126 110.000003) (width 0.25) (layer "B.Cu") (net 14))
 (segment (start 132.27787 110.870839) (end 132.248709 110.9) (width 0.25) (layer "F.Cu") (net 17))
 (segment (start 132.248709 110.9) (end 128.1 110.9) (width 0.25) (layer "F.Cu") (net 17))
 (via (at 132.27787 110.870839) (size 0.8) (drill 0.4) (layers "F.Cu" "B.Cu") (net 17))
 (segment (start 147.875153 116.524847) (end 146.081802 114.731496) (width 0.25) (layer "B.Cu") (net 17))
 (segment (start 160.418198 116.225) (end 160.418198 115.6) (width 0.2) (layer "B.Cu") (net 17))
 (segment (start 143.540812 109.55) (end 141.713604 109.55) (width 0.25) (layer "B.Cu") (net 17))
 (segment (start 149.725306 118.375) (end 147.875153 116.524847) (width 0.25) (layer "B.Cu") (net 17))
 (segment (start 145.445406 111.454594) (end 143.540812 109.55) (width 0.25) (layer "B.Cu") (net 17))
 (segment (start 141.713604 109.55) (end 133.598709 109.55) (width 0.25) (layer "B.Cu") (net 17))
 (segment (start 146.081802 114.731496) (end 146.081802 113.3) (width 0.25) (layer "B.Cu") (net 17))
 (segment (start 146.081802 112.09099) (end 145.445406 111.454594) (width 0.25) (layer "B.Cu") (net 17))
 (segment (start 146.081802 113.3) (end 146.081802 112.09099) (width 0.25) (layer "B.Cu") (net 17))
 (segment (start 133.598709 109.55) (end 132.27787 110.870839) (width 0.25) (layer "B.Cu") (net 17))
 (segment (start 124.800006 111.000006) (end 124.7 110.9) (width 0.25) (layer "F.Cu") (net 16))
 (segment (start 126 111.000006) (end 124.800006 111.000006) (width 0.25) (layer "F.Cu") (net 16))
 (via (at 126 111.000006) (size 0.8) (drill 0.4) (layers "F.Cu" "B.Cu") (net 16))
 (segment (start 146.531802 114.5451) (end 146.531802 111.904594) (width 0.25) (layer "B.Cu") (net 16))
 (segment (start 146.531802 111.904594) (end 143.727208 109.1) (width 0.25) (layer "B.Cu") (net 16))
 (segment (start 149.911702 117.925) (end 146.531802 114.5451) (width 0.25) (layer "B.Cu") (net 16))
 (segment (start 133.023403 109.1) (end 131.123397 111.000006) (width 0.25) (layer "B.Cu") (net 16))
 (segment (start 131.123397 111.000006) (end 126 111.000006) (width 0.25) (layer "B.Cu") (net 16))
 (segment (start 143.727208 109.1) (end 133.023403 109.1) (width 0.25) (layer "B.Cu") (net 16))
 (segment (start 133.712653 111.712653) (end 133.7 111.7) (width 0.25) (layer "F.Cu") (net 19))
 (segment (start 133.7 111.7) (end 128.1 111.7) (width 0.25) (layer "F.Cu") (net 19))
 (via (at 133.712653 111.712653) (size 0.8) (drill 0.4) (layers "F.Cu" "B.Cu") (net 19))
 (segment (start 145.181802 112.463782) (end 144.70901 111.99099) (width 0.25) (layer "B.Cu") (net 19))
 (segment (start 148.438757 118.361243) (end 145.181802 115.104288) (width 0.25) (layer "B.Cu") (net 19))
 (segment (start 134.975306 110.45) (end 133.712653 111.712653) (width 0.25) (layer "B.Cu") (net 19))
 (segment (start 144.70901 111.99099) (end 143.16802 110.45) (width 0.25) (layer "B.Cu") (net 19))
 (segment (start 145.181802 115.104288) (end 145.181802 113.9) (width 0.25) (layer "B.Cu") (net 19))
 (segment (start 149.352514 119.275) (end 148.438757 118.361243) (width 0.25) (layer "B.Cu") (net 19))
 (segment (start 145.181802 113.9) (end 145.181802 112.463782) (width 0.25) (layer "B.Cu") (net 19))
 (segment (start 141 110.45) (end 134.975306 110.45) (width 0.25) (layer "B.Cu") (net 19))
 (segment (start 143.16802 110.45) (end 141 110.45) (width 0.25) (layer "B.Cu") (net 19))
 (segment (start 125.699991 111.7) (end 124.7 111.7) (width 0.25) (layer "F.Cu") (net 18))
 (segment (start 126 112.000009) (end 125.699991 111.7) (width 0.25) (layer "F.Cu") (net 18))
 (via (at 126 112.000009) (size 0.8) (drill 0.4) (layers "F.Cu" "B.Cu") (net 18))
 (segment (start 134.4 110) (end 132.399991 112.000009) (width 0.25) (layer "B.Cu") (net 18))
 (segment (start 145.631802 114.5451) (end 145.631802 112.277386) (width 0.25) (layer "B.Cu") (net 18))
 (segment (start 149.53891 118.825) (end 149.275306 118.561396) (width 0.25) (layer "B.Cu") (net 18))
 (segment (start 145.631802 114.917892) (end 145.631802 114.5451) (width 0.25) (layer "B.Cu") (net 18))
 (segment (start 149.275306 118.561396) (end 145.631802 114.917892) (width 0.25) (layer "B.Cu") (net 18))
 (segment (start 132.399991 112.000009) (end 126 112.000009) (width 0.25) (layer "B.Cu") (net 18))
 (segment (start 143.354416 110) (end 140.8 110) (width 0.25) (layer "B.Cu") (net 18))
 (segment (start 135.3 110) (end 134.4 110) (width 0.25) (layer "B.Cu") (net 18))
 (segment (start 144.677208 111.322792) (end 143.354416 110) (width 0.25) (layer "B.Cu") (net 18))
 (segment (start 145.631802 112.277386) (end 144.677208 111.322792) (width 0.25) (layer "B.Cu") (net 18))
 (segment (start 140.8 110) (end 135.3 110) (width 0.25) (layer "B.Cu") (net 18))
 (segment (start 126.4 113.4) (end 127.2 113.4) (width 0.25) (layer "F.Cu") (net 3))
 (segment (start 145 105) (end 143.65 105) (width 0.2) (layer "F.Cu") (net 3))
 (segment (start 142.35 106.3) (end 142.35 108.5) (width 0.2) (layer "F.Cu") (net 3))
 (segment (start 115 104) (end 112.5 106.5) (width 0.25) (layer "F.Cu") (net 3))
 (segment (start 134.9 105.675) (end 134.9 111.550611) (width 0.25) (layer "F.Cu") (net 3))
 (segment (start 113.9 113.4) (end 125.6 113.4) (width 0.25) (layer "F.Cu") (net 3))
 (segment (start 134.9 111.550611) (end 133.050611 113.4) (width 0.25) (layer "F.Cu") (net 3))
 (segment (start 133.050611 113.4) (end 127.2 113.4) (width 0.25) (layer "F.Cu") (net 3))
 (segment (start 143 108.5) (end 142.35 108.5) (width 0.2) (layer "F.Cu") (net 3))
 (segment (start 112.5 112) (end 113.9 113.4) (width 0.25) (layer "F.Cu") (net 3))
 (segment (start 112.5 106.5) (end 112.5 112) (width 0.25) (layer "F.Cu") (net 3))
 (segment (start 124.7 112.5) (end 125.6 113.4) (width 0.25) (layer "F.Cu") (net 3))
 (segment (start 125.6 113.4) (end 126.4 113.4) (width 0.25) (layer "F.Cu") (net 3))
 (segment (start 143.65 105) (end 142.35 106.3) (width 0.2) (layer "F.Cu") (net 3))
 (segment (start 144.9 105.1) (end 145 105) (width 0.2) (layer "F.Cu") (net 3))
 (segment (start 127.2 113.4) (end 128.1 112.5) (width 0.25) (layer "F.Cu") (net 3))
 (via (at 145 105) (size 0.6) (drill 0.3) (layers "F.Cu" "B.Cu") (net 3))
 (via (at 134.9 105.675) (size 0.8) (drill 0.4) (layers "F.Cu" "B.Cu") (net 3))
 (segment (start 145 105.95) (end 135.175 105.95) (width 0.25) (layer "B.Cu") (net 3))
 (segment (start 145 105) (end 145 105.95) (width 0.2) (layer "B.Cu") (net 3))
 (segment (start 135.175 105.95) (end 134.9 105.675) (width 0.25) (layer "B.Cu") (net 3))
 (segment (start 145.601 104.751057) (end 142.748943 101.899) (width 0.2) (layer "F.Cu") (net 2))
 (segment (start 122.181 101.899) (end 115 109.08) (width 0.2) (layer "F.Cu") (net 2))
 (segment (start 145.601 105.248943) (end 145.601 104.751057) (width 0.2) (layer "F.Cu") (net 2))
 (segment (start 142.748943 101.899) (end 122.181 101.899) (width 0.2) (layer "F.Cu") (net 2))
 (segment (start 143.65 106.3) (end 144.549943 106.3) (width 0.2) (layer "F.Cu") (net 2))
 (segment (start 144.549943 106.3) (end 145.601 105.248943) (width 0.2) (layer "F.Cu") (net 2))
 (segment (start 116.96 106.54) (end 115 106.54) (width 0.2) (layer "F.Cu") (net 1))
 (segment (start 143.65 108.5) (end 146.002 106.148) (width 0.2) (layer "F.Cu") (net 1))
 (segment (start 142.915043 101.498) (end 122.002 101.498) (width 0.2) (layer "F.Cu") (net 1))
 (segment (start 146.002 104.584957) (end 142.915043 101.498) (width 0.2) (layer "F.Cu") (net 1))
 (segment (start 122.002 101.498) (end 116.96 106.54) (width 0.2) (layer "F.Cu") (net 1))
 (segment (start 146.002 106.148) (end 146.002 104.584957) (width 0.2) (layer "F.Cu") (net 1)))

